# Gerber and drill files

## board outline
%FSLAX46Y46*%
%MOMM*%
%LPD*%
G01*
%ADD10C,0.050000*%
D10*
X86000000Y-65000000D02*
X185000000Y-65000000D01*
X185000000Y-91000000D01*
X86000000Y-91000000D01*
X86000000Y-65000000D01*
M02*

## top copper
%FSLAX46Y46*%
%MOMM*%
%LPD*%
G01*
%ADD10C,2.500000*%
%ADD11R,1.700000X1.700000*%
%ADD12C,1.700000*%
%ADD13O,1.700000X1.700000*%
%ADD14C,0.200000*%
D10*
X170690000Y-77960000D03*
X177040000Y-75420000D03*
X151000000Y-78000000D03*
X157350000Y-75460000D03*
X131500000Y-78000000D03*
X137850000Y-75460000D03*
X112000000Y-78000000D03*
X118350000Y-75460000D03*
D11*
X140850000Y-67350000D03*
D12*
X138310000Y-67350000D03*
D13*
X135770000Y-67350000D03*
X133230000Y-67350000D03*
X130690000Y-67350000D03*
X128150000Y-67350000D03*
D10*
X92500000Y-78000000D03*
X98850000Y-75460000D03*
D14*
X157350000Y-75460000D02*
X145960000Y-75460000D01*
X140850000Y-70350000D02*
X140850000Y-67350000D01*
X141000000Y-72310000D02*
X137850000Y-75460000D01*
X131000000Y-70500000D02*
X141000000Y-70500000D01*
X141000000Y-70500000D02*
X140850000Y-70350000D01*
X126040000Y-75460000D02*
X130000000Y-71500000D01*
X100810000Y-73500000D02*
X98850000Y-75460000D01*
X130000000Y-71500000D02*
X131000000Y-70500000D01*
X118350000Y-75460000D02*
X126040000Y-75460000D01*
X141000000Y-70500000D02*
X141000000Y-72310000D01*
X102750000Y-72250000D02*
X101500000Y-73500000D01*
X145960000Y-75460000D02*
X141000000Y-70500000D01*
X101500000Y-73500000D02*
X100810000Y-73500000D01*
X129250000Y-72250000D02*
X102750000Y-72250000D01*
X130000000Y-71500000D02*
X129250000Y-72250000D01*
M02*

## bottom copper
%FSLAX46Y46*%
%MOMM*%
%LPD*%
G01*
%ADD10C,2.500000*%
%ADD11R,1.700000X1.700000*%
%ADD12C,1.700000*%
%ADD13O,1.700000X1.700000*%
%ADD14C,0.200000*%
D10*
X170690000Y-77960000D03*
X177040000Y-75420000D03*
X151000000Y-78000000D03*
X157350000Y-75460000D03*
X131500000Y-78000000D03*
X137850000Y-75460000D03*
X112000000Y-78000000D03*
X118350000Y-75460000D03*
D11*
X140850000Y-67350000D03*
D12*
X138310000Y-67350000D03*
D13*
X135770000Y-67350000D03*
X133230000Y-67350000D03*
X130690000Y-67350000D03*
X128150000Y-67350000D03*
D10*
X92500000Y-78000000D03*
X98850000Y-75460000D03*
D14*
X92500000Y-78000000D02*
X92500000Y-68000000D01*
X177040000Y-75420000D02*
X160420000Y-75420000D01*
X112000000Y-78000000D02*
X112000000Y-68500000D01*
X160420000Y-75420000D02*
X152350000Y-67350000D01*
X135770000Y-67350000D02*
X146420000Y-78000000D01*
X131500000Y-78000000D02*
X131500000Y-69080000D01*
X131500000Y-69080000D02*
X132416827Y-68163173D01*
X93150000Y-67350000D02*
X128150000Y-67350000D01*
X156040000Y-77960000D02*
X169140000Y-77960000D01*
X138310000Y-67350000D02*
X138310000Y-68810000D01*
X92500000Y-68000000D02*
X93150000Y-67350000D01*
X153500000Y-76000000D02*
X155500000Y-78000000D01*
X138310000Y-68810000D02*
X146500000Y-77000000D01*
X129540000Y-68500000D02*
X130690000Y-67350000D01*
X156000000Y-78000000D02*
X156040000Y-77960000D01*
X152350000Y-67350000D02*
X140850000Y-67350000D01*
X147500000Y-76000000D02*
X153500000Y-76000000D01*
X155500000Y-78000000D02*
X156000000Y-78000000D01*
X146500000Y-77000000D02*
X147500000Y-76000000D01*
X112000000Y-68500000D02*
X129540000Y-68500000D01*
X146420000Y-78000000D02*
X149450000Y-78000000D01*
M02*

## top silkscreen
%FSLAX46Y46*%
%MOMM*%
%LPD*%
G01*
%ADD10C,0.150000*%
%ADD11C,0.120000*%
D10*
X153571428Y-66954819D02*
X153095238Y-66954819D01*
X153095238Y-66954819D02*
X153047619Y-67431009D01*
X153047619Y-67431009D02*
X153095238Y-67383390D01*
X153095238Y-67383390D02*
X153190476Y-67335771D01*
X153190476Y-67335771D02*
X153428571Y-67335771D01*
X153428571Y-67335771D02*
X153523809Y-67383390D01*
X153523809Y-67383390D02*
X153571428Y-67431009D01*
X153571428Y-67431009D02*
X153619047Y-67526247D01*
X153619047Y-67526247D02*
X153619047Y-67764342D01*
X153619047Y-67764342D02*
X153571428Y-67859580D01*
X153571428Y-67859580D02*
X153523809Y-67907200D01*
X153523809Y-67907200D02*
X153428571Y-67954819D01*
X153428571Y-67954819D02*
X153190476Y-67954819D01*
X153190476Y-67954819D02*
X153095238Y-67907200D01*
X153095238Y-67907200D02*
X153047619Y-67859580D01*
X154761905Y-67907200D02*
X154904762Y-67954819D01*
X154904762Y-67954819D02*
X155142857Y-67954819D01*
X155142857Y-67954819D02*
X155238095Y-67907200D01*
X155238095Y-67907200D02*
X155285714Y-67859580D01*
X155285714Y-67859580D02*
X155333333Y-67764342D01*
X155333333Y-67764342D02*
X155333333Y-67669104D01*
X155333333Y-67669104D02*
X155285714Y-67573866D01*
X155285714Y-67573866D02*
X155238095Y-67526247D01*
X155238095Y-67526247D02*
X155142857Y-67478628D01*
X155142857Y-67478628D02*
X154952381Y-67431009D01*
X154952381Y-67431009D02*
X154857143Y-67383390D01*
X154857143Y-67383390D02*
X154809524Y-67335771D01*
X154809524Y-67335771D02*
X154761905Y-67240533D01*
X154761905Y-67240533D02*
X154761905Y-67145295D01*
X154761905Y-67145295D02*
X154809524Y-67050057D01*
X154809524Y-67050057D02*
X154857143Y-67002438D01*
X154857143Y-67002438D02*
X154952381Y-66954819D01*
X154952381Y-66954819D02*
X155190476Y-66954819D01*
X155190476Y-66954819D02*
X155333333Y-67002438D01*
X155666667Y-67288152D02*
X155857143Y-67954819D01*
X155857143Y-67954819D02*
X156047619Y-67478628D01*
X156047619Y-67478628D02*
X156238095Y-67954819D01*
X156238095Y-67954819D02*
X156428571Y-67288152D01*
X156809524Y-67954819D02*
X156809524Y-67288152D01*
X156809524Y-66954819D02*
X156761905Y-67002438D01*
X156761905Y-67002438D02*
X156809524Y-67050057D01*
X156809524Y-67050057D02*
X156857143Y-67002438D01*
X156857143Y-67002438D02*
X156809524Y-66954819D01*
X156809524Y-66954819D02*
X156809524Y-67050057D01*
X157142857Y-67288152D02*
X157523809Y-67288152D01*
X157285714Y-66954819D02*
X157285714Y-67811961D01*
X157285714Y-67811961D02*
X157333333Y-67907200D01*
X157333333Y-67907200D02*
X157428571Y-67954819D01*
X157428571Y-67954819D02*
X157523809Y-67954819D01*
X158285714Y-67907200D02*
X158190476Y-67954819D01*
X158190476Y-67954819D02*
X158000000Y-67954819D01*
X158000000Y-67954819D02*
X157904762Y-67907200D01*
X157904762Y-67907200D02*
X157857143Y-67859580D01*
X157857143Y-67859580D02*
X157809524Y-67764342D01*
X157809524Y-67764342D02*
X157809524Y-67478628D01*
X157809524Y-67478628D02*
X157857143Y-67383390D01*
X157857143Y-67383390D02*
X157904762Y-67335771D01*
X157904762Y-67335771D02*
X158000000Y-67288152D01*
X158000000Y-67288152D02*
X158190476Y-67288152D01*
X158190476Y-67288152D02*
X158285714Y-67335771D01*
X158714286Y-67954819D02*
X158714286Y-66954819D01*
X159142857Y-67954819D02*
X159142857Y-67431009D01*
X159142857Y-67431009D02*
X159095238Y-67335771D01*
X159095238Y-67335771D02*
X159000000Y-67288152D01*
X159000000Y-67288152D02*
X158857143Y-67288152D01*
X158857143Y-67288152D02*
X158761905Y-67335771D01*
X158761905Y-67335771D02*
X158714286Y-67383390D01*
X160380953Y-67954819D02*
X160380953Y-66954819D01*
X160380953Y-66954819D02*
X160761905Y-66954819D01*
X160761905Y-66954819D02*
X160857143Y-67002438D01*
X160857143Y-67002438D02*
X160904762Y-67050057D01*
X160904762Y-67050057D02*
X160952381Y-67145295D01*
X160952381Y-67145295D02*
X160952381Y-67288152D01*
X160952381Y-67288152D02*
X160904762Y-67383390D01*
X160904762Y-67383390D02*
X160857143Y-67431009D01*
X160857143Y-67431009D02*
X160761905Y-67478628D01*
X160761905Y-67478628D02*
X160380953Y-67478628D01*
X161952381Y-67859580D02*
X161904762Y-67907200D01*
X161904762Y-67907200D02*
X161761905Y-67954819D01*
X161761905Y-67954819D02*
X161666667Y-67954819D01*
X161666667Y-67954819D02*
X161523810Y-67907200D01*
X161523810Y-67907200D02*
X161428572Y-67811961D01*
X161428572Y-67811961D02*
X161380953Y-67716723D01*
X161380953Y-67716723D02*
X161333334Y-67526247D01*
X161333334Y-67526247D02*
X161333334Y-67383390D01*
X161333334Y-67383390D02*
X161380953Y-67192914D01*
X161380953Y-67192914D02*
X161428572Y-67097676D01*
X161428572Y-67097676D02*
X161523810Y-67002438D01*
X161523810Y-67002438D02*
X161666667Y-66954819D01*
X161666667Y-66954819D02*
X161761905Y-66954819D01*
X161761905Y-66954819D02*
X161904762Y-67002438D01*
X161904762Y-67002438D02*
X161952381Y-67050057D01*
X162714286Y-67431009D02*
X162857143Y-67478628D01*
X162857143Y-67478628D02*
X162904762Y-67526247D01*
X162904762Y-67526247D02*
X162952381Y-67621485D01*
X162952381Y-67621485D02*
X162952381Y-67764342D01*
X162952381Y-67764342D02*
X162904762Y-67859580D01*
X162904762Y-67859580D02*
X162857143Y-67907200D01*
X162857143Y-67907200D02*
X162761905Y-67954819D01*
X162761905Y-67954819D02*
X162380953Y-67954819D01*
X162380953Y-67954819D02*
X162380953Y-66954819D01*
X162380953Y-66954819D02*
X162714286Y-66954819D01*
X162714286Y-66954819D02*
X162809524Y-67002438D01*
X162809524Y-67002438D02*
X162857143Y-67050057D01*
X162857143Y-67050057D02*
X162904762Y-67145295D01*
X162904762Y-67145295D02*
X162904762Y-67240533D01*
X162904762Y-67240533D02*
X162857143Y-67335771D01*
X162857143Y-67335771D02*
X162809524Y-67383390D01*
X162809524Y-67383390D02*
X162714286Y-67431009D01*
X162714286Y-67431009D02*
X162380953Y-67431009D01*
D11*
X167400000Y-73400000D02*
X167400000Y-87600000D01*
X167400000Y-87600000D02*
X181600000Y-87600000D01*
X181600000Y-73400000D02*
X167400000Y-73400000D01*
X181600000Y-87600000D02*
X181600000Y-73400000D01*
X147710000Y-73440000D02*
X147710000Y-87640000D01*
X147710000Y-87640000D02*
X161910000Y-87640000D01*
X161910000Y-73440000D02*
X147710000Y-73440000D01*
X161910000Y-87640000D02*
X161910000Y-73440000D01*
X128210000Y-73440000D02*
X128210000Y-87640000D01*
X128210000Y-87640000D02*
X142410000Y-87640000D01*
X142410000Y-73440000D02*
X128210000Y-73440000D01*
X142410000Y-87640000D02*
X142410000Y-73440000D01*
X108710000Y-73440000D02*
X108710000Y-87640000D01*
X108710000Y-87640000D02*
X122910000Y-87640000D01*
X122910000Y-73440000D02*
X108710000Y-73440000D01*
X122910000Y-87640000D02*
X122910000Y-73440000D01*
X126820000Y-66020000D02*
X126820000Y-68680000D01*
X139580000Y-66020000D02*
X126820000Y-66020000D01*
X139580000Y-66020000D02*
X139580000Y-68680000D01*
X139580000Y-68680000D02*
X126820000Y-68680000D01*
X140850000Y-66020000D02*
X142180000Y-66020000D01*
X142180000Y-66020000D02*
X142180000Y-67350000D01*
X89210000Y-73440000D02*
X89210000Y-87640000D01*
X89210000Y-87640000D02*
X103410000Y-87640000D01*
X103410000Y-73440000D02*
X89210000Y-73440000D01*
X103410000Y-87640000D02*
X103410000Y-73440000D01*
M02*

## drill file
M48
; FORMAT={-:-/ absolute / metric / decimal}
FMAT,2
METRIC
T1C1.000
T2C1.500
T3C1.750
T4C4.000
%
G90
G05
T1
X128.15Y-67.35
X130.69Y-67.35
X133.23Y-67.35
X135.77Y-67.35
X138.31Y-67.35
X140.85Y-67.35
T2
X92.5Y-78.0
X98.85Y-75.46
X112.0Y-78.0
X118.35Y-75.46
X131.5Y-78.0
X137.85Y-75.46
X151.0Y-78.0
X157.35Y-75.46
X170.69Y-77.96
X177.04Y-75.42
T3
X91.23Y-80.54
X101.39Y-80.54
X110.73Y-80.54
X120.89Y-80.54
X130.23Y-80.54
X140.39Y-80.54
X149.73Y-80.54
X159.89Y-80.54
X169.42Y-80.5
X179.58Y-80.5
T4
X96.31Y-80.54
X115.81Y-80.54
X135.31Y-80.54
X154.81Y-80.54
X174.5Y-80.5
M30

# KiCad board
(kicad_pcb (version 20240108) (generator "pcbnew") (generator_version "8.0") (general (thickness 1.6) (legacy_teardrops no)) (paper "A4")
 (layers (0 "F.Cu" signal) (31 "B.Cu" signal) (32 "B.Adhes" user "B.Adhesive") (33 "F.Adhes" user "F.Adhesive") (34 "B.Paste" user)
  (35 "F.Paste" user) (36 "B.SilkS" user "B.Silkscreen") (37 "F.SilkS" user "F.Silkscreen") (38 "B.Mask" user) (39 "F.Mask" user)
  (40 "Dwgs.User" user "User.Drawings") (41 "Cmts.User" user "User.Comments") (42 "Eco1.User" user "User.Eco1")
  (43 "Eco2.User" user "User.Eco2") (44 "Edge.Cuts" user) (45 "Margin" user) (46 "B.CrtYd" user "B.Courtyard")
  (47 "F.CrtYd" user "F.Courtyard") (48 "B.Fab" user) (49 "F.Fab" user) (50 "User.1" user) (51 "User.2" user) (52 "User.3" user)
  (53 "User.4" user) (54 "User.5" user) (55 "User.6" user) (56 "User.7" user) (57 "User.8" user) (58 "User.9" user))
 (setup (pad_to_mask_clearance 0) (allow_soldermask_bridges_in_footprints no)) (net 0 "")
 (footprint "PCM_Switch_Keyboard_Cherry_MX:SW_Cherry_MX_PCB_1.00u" (layer "F.Cu") (at 174.5 80.5)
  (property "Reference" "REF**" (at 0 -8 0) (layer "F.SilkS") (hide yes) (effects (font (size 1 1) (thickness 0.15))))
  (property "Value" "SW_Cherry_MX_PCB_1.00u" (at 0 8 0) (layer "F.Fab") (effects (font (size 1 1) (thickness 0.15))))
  (fp_line (start -7.1 -7.1) (end -7.1 7.1) (stroke (width 0.12) (type solid)) (layer "F.SilkS"))
  (fp_line (start -7.1 7.1) (end 7.1 7.1) (stroke (width 0.12) (type solid)) (layer "F.SilkS"))
  (fp_line (start 7.1 -7.1) (end -7.1 -7.1) (stroke (width 0.12) (type solid)) (layer "F.SilkS"))
  (fp_line (start 7.1 7.1) (end 7.1 -7.1) (stroke (width 0.12) (type solid)) (layer "F.SilkS"))
  (pad "" np_thru_hole circle (at -5.08 0) (size 1.75 1.75) (drill 1.75) (layers "F&B.Cu" "*.Mask"))
  (pad "" np_thru_hole circle (at 0 0) (size 4 4) (drill 4) (layers "F&B.Cu" "*.Mask"))
  (pad "" np_thru_hole circle (at 5.08 0) (size 1.75 1.75) (drill 1.75) (layers "F&B.Cu" "*.Mask"))
  (pad "1" thru_hole circle (at -3.81 -2.54) (size 2.5 2.5) (drill 1.5) (layers "*.Cu" "*.Mask") (remove_unused_layers no))
  (pad "2" thru_hole circle (at 2.54 -5.08) (size 2.5 2.5) (drill 1.5) (layers "*.Cu" "*.Mask") (remove_unused_layers no)))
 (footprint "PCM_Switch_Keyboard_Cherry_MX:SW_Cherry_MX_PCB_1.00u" (layer "F.Cu") (at 154.81 80.54)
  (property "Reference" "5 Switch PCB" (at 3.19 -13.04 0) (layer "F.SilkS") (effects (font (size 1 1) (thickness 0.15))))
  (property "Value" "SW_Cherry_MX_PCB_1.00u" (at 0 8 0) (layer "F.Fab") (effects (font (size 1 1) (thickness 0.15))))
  (fp_line (start -7.1 -7.1) (end -7.1 7.1) (stroke (width 0.12) (type solid)) (layer "F.SilkS"))
  (fp_line (start -7.1 7.1) (end 7.1 7.1) (stroke (width 0.12) (type solid)) (layer "F.SilkS"))
  (fp_line (start 7.1 -7.1) (end -7.1 -7.1) (stroke (width 0.12) (type solid)) (layer "F.SilkS"))
  (fp_line (start 7.1 7.1) (end 7.1 -7.1) (stroke (width 0.12) (type solid)) (layer "F.SilkS"))
  (pad "" np_thru_hole circle (at -5.08 0) (size 1.75 1.75) (drill 1.75) (layers "F&B.Cu" "*.Mask"))
  (pad "" np_thru_hole circle (at 0 0) (size 4 4) (drill 4) (layers "F&B.Cu" "*.Mask"))
  (pad "" np_thru_hole circle (at 5.08 0) (size 1.75 1.75) (drill 1.75) (layers "F&B.Cu" "*.Mask"))
  (pad "1" thru_hole circle (at -3.81 -2.54) (size 2.5 2.5) (drill 1.5) (layers "*.Cu" "*.Mask") (remove_unused_layers no))
  (pad "2" thru_hole circle (at 2.54 -5.08) (size 2.5 2.5) (drill 1.5) (layers "*.Cu" "*.Mask") (remove_unused_layers no)))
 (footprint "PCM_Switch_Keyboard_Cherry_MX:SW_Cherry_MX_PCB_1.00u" (layer "F.Cu") (at 135.31 80.54)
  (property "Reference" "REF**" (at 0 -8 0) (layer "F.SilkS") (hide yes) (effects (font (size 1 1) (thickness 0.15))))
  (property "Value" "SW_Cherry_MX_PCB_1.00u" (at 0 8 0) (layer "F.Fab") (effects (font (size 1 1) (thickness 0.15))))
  (fp_line (start -7.1 -7.1) (end -7.1 7.1) (stroke (width 0.12) (type solid)) (layer "F.SilkS"))
  (fp_line (start -7.1 7.1) (end 7.1 7.1) (stroke (width 0.12) (type solid)) (layer "F.SilkS"))
  (fp_line (start 7.1 -7.1) (end -7.1 -7.1) (stroke (width 0.12) (type solid)) (layer "F.SilkS"))
  (fp_line (start 7.1 7.1) (end 7.1 -7.1) (stroke (width 0.12) (type solid)) (layer "F.SilkS"))
  (pad "" np_thru_hole circle (at -5.08 0) (size 1.75 1.75) (drill 1.75) (layers "F&B.Cu" "*.Mask"))
  (pad "" np_thru_hole circle (at 0 0) (size 4 4) (drill 4) (layers "F&B.Cu" "*.Mask"))
  (pad "" np_thru_hole circle (at 5.08 0) (size 1.75 1.75) (drill 1.75) (layers "F&B.Cu" "*.Mask"))
  (pad "1" thru_hole circle (at -3.81 -2.54) (size 2.5 2.5) (drill 1.5) (layers "*.Cu" "*.Mask") (remove_unused_layers no))
  (pad "2" thru_hole circle (at 2.54 -5.08) (size 2.5 2.5) (drill 1.5) (layers "*.Cu" "*.Mask") (remove_unused_layers no)))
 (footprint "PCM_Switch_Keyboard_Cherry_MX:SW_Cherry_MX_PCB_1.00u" (layer "F.Cu") (at 115.81 80.54)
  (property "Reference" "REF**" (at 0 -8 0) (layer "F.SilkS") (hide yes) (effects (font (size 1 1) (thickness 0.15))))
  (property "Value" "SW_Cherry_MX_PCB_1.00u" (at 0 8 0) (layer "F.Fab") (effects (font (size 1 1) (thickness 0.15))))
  (fp_line (start -7.1 -7.1) (end -7.1 7.1) (stroke (width 0.12) (type solid)) (layer "F.SilkS"))
  (fp_line (start -7.1 7.1) (end 7.1 7.1) (stroke (width 0.12) (type solid)) (layer "F.SilkS"))
  (fp_line (start 7.1 -7.1) (end -7.1 -7.1) (stroke (width 0.12) (type solid)) (layer "F.SilkS"))
  (fp_line (start 7.1 7.1) (end 7.1 -7.1) (stroke (width 0.12) (type solid)) (layer "F.SilkS"))
  (pad "" np_thru_hole circle (at -5.08 0) (size 1.75 1.75) (drill 1.75) (layers "*.Cu" "*.Mask"))
  (pad "" np_thru_hole circle (at 0 0) (size 4 4) (drill 4) (layers "*.Cu" "*.Mask"))
  (pad "" np_thru_hole circle (at 5.08 0) (size 1.75 1.75) (drill 1.75) (layers "*.Cu" "*.Mask"))
  (pad "1" thru_hole circle (at -3.81 -2.54) (size 2.5 2.5) (drill 1.5) (layers "*.Cu" "*.Mask") (remove_unused_layers no))
  (pad "2" thru_hole circle (at 2.54 -5.08) (size 2.5 2.5) (drill 1.5) (layers "*.Cu" "*.Mask") (remove_unused_layers no)))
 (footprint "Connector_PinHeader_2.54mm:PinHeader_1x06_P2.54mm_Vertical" (layer "F.Cu") (at 140.85 67.35 -90)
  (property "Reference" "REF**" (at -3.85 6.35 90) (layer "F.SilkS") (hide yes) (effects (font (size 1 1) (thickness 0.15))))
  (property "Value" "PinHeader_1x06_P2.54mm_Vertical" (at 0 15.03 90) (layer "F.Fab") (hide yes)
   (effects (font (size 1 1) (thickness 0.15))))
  (fp_line (start -1.33 14.03) (end 1.33 14.03) (stroke (width 0.12) (type solid)) (layer "F.SilkS"))
  (fp_line (start -1.33 1.27) (end -1.33 14.03) (stroke (width 0.12) (type solid)) (layer "F.SilkS"))
  (fp_line (start -1.33 1.27) (end 1.33 1.27) (stroke (width 0.12) (type solid)) (layer "F.SilkS"))
  (fp_line (start 1.33 1.27) (end 1.33 14.03) (stroke (width 0.12) (type solid)) (layer "F.SilkS"))
  (fp_line (start -1.33 0) (end -1.33 -1.33) (stroke (width 0.12) (type solid)) (layer "F.SilkS"))
  (fp_line (start -1.33 -1.33) (end 0 -1.33) (stroke (width 0.12) (type solid)) (layer "F.SilkS"))
  (pad "1" thru_hole rect (at 0 0 270) (size 1.7 1.7) (drill 1) (layers "*.Cu" "*.Mask") (remove_unused_layers no))
  (pad "2" thru_hole circle (at 0 2.54 270) (size 1.7 1.7) (drill 1) (layers "*.Cu" "*.Mask") (remove_unused_layers no))
  (pad "3" thru_hole oval (at 0 5.08 270) (size 1.7 1.7) (drill 1) (layers "*.Cu" "*.Mask") (remove_unused_layers no))
  (pad "4" thru_hole oval (at 0 7.62 270) (size 1.7 1.7) (drill 1) (layers "*.Cu" "*.Mask") (remove_unused_layers no))
  (pad "5" thru_hole oval (at 0 10.16 270) (size 1.7 1.7) (drill 1) (layers "*.Cu" "*.Mask") (remove_unused_layers no))
  (pad "6" thru_hole oval (at 0 12.7 270) (size 1.7 1.7) (drill 1) (layers "*.Cu" "*.Mask") (remove_unused_layers no)))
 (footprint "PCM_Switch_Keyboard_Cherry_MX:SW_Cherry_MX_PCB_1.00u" (layer "F.Cu") (at 96.31 80.54)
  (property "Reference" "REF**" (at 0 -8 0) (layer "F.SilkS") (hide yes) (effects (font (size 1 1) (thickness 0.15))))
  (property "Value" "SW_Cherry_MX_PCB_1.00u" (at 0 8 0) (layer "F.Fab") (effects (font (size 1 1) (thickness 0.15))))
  (fp_line (start -7.1 -7.1) (end -7.1 7.1) (stroke (width 0.12) (type solid)) (layer "F.SilkS"))
  (fp_line (start -7.1 7.1) (end 7.1 7.1) (stroke (width 0.12) (type solid)) (layer "F.SilkS"))
  (fp_line (start 7.1 -7.1) (end -7.1 -7.1) (stroke (width 0.12) (type solid)) (layer "F.SilkS"))
  (fp_line (start 7.1 7.1) (end 7.1 -7.1) (stroke (width 0.12) (type solid)) (layer "F.SilkS"))
  (pad "" np_thru_hole circle (at -5.08 0) (size 1.75 1.75) (drill 1.75) (layers "F&B.Cu" "*.Mask"))
  (pad "" np_thru_hole circle (at 0 0) (size 4 4) (drill 4) (layers "F&B.Cu" "*.Mask"))
  (pad "" np_thru_hole circle (at 5.08 0) (size 1.75 1.75) (drill 1.75) (layers "F&B.Cu" "*.Mask"))
  (pad "1" thru_hole circle (at -3.81 -2.54) (size 2.5 2.5) (drill 1.5) (layers "*.Cu" "*.Mask") (remove_unused_layers no))
  (pad "2" thru_hole circle (at 2.54 -5.08) (size 2.5 2.5) (drill 1.5) (layers "*.Cu" "*.Mask") (remove_unused_layers no)))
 (gr_rect (start 86 65) (end 185 91) (stroke (width 0.05) (type default)) (fill none) (layer "Edge.Cuts"))
 (segment (start 157.35 75.46) (end 145.96 75.46) (width 0.2) (layer "F.Cu") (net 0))
 (segment (start 140.85 70.35) (end 140.85 67.35) (width 0.2) (layer "F.Cu") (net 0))
 (segment (start 141 72.31) (end 137.85 75.46) (width 0.2) (layer "F.Cu") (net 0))
 (segment (start 131 70.5) (end 141 70.5) (width 0.2) (layer "F.Cu") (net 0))
 (segment (start 141 70.5) (end 140.85 70.35) (width 0.2) (layer "F.Cu") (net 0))
 (segment (start 126.04 75.46) (end 130 71.5) (width 0.2) (layer "F.Cu") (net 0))
 (segment (start 100.81 73.5) (end 98.85 75.46) (width 0.2) (layer "F.Cu") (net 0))
 (segment (start 130 71.5) (end 131 70.5) (width 0.2) (layer "F.Cu") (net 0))
 (segment (start 118.35 75.46) (end 126.04 75.46) (width 0.2) (layer "F.Cu") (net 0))
 (segment (start 141 70.5) (end 141 72.31) (width 0.2) (layer "F.Cu") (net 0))
 (segment (start 102.75 72.25) (end 101.5 73.5) (width 0.2) (layer "F.Cu") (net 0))
 (segment (start 145.96 75.46) (end 141 70.5) (width 0.2) (layer "F.Cu") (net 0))
 (segment (start 101.5 73.5) (end 100.81 73.5) (width 0.2) (layer "F.Cu") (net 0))
 (segment (start 129.25 72.25) (end 102.75 72.25) (width 0.2) (layer "F.Cu") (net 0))
 (segment (start 130 71.5) (end 129.25 72.25) (width 0.2) (layer "F.Cu") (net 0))
 (segment (start 92.5 78) (end 92.5 68) (width 0.2) (layer "B.Cu") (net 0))
 (segment (start 177.04 75.42) (end 160.42 75.42) (width 0.2) (layer "B.Cu") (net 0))
 (segment (start 112 78) (end 112 68.5) (width 0.2) (layer "B.Cu") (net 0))
 (segment (start 160.42 75.42) (end 152.35 67.35) (width 0.2) (layer "B.Cu") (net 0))
 (segment (start 135.77 67.35) (end 146.42 78) (width 0.2) (layer "B.Cu") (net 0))
 (segment (start 131.5 78) (end 131.5 69.08) (width 0.2) (layer "B.Cu") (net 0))
 (segment (start 131.5 69.08) (end 132.416827 68.163173) (width 0.2) (layer "B.Cu") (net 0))
 (segment (start 93.15 67.35) (end 128.15 67.35) (width 0.2) (layer "B.Cu") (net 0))
 (segment (start 156.04 77.96) (end 169.14 77.96) (width 0.2) (layer "B.Cu") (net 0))
 (segment (start 138.31 67.35) (end 138.31 68.81) (width 0.2) (layer "B.Cu") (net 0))
 (segment (start 92.5 68) (end 93.15 67.35) (width 0.2) (layer "B.Cu") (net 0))
 (segment (start 153.5 76) (end 155.5 78) (width 0.2) (layer "B.Cu") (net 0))
 (segment (start 138.31 68.81) (end 146.5 77) (width 0.2) (layer "B.Cu") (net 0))
 (segment (start 129.54 68.5) (end 130.69 67.35) (width 0.2) (layer "B.Cu") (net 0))
 (segment (start 156 78) (end 156.04 77.96) (width 0.2) (layer "B.Cu") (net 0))
 (segment (start 152.35 67.35) (end 140.85 67.35) (width 0.2) (layer "B.Cu") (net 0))
 (segment (start 147.5 76) (end 153.5 76) (width 0.2) (layer "B.Cu") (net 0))
 (segment (start 155.5 78) (end 156 78) (width 0.2) (layer "B.Cu") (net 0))
 (segment (start 146.5 77) (end 147.5 76) (width 0.2) (layer "B.Cu") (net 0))
 (segment (start 112 68.5) (end 129.54 68.5) (width 0.2) (layer "B.Cu") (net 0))
 (segment (start 146.42 78) (end 149.45 78) (width 0.2) (layer "B.Cu") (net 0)))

